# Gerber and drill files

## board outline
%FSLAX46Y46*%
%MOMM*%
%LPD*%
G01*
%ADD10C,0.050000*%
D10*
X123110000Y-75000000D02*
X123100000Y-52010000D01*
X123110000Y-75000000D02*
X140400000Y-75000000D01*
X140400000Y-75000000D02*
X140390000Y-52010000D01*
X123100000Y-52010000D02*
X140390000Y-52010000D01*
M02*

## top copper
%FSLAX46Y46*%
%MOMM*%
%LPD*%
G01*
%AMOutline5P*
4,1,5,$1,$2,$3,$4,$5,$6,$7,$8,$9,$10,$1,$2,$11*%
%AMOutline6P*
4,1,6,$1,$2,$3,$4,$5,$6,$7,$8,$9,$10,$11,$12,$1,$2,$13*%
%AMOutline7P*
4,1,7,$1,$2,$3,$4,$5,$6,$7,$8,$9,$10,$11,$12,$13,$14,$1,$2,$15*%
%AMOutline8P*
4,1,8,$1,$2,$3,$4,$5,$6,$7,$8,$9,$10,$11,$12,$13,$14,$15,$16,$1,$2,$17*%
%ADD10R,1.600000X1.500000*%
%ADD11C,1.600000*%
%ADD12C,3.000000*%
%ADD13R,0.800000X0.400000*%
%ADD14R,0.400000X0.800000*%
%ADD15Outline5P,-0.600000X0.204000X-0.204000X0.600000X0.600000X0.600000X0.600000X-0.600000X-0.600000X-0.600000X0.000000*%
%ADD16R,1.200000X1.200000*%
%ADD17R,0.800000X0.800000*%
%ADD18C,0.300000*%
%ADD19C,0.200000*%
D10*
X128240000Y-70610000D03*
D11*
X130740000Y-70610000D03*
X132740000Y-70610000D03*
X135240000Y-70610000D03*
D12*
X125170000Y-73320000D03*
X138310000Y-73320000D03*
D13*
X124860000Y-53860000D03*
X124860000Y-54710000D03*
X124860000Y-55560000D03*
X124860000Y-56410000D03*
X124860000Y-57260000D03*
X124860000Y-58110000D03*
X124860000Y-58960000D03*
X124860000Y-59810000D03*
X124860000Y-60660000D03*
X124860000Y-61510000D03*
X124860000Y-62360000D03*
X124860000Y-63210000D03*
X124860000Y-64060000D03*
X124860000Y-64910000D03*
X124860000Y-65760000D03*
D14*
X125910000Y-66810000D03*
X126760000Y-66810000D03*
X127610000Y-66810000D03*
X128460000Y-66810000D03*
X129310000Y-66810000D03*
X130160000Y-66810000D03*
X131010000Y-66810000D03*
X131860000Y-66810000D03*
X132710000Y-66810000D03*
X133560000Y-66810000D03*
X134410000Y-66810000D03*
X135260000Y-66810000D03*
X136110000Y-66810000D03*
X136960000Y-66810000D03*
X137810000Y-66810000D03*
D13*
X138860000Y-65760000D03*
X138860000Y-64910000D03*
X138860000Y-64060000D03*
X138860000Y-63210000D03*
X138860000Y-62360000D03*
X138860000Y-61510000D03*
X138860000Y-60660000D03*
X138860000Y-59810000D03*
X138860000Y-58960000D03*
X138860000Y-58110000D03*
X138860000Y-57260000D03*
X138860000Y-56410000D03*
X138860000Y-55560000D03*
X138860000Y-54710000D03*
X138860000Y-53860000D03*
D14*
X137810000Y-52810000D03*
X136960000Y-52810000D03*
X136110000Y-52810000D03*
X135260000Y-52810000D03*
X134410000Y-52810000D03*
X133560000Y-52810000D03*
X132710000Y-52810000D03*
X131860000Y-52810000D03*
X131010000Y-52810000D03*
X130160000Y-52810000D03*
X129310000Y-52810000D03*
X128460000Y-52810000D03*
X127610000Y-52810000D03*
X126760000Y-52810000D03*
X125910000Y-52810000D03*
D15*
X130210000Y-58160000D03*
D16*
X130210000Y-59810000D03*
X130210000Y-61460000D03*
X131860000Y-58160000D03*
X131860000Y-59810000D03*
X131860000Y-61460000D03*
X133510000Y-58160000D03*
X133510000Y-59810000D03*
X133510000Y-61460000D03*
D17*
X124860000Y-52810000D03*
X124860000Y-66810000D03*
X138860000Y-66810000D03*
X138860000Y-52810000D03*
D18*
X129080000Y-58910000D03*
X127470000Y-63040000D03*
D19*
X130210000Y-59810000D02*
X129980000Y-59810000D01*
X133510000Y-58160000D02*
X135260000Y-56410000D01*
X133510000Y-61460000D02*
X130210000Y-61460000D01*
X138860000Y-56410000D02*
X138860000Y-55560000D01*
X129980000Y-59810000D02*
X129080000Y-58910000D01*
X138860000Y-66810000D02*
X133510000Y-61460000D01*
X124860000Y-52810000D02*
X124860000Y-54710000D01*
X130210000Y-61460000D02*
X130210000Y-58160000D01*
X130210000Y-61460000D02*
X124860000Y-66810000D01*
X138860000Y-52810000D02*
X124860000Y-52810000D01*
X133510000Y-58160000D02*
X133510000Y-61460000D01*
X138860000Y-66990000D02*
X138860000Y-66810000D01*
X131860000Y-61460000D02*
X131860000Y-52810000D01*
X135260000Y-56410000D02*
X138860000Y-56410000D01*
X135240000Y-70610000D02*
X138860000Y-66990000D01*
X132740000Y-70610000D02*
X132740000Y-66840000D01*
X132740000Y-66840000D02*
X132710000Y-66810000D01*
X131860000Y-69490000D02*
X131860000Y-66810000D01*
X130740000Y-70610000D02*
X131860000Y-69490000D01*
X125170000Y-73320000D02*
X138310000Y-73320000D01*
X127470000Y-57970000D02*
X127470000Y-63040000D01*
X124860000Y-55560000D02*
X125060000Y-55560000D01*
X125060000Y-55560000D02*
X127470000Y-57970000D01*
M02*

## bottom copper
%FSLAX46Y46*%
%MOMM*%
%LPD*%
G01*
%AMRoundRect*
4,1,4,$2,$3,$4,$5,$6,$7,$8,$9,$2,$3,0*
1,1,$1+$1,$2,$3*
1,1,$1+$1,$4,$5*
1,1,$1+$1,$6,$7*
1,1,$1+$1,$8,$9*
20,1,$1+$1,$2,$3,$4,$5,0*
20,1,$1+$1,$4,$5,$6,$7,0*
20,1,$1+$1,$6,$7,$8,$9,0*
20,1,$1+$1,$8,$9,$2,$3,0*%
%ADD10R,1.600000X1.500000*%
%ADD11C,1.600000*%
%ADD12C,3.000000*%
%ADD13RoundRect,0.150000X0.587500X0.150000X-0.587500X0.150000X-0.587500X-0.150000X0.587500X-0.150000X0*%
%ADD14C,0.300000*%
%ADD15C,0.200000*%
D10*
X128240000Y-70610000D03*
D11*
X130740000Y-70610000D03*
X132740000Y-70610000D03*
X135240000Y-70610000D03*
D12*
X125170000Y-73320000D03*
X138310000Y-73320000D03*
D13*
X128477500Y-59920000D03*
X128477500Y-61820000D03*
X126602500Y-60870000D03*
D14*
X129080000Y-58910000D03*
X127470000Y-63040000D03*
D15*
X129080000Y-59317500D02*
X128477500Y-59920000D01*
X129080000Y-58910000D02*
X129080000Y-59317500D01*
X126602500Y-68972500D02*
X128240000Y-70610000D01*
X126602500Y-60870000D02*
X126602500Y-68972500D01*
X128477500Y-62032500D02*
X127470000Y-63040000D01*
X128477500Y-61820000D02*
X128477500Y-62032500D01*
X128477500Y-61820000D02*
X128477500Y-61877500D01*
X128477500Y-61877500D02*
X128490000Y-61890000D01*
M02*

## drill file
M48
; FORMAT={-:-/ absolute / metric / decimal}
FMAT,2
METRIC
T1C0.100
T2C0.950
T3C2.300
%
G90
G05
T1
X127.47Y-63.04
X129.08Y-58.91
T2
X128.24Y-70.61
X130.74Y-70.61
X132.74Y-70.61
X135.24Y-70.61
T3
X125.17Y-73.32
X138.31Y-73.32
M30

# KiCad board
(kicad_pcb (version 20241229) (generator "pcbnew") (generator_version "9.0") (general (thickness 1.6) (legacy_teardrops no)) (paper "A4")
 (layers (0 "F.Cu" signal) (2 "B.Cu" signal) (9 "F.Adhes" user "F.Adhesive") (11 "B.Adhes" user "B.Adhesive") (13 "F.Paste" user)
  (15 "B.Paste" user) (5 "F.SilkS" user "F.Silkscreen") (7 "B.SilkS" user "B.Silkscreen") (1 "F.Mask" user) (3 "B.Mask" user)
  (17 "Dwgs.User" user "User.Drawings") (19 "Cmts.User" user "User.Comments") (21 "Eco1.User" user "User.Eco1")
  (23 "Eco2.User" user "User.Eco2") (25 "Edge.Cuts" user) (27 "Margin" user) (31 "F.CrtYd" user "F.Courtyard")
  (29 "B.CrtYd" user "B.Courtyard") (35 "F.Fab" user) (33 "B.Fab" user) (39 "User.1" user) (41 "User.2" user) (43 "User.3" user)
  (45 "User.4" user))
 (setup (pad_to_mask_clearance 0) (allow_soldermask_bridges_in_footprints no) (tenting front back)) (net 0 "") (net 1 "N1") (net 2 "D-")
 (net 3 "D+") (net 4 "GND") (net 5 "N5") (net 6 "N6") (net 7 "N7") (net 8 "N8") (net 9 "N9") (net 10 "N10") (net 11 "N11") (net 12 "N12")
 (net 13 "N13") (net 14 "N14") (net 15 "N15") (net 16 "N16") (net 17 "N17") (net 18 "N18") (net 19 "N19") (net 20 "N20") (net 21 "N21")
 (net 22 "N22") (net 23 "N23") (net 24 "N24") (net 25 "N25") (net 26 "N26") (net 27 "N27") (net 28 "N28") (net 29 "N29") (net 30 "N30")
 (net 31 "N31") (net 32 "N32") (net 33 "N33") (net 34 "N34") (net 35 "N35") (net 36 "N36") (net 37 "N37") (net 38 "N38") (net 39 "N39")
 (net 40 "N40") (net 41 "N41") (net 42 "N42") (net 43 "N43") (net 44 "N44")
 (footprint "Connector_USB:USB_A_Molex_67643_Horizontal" (layer "F.Cu") (at 128.24 70.61)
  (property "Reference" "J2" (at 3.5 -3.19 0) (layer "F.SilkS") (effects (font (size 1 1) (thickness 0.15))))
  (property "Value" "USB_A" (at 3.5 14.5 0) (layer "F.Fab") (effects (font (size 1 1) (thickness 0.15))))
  (pad "1" thru_hole rect (at 0 0) (size 1.6 1.5) (drill 0.95) (layers "*.Cu" "*.Mask") (remove_unused_layers no) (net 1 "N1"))
  (pad "2" thru_hole circle (at 2.5 0) (size 1.6 1.6) (drill 0.95) (layers "*.Cu" "*.Mask") (remove_unused_layers no) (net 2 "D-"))
  (pad "3" thru_hole circle (at 4.5 0) (size 1.6 1.6) (drill 0.95) (layers "*.Cu" "*.Mask") (remove_unused_layers no) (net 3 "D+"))
  (pad "4" thru_hole circle (at 7 0) (size 1.6 1.6) (drill 0.95) (layers "*.Cu" "*.Mask") (remove_unused_layers no) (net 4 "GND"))
  (pad "5" thru_hole circle (at -3.07 2.71) (size 3 3) (drill 2.3) (layers "*.Cu" "*.Mask") (remove_unused_layers no) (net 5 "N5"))
  (pad "5" thru_hole circle (at 10.07 2.71) (size 3 3) (drill 2.3) (layers "*.Cu" "*.Mask") (remove_unused_layers no) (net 5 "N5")))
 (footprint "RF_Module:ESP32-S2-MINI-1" (layer "F.Cu") (at 131.86 57.26)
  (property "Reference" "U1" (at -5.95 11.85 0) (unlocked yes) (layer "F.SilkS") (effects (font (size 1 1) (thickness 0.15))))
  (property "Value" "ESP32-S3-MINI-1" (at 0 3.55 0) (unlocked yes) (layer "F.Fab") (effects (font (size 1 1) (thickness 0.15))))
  (pad "1" smd rect (at -7 -3.4) (size 0.8 0.4) (layers "F.Cu" "F.Mask" "F.Paste") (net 4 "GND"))
  (pad "2" smd rect (at -7 -2.55) (size 0.8 0.4) (layers "F.Cu" "F.Mask" "F.Paste") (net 4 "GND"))
  (pad "3" smd rect (at -7 -1.7) (size 0.8 0.4) (layers "F.Cu" "F.Mask" "F.Paste") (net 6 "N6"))
  (pad "4" smd rect (at -7 -0.85) (size 0.8 0.4) (layers "F.Cu" "F.Mask" "F.Paste") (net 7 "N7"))
  (pad "5" smd rect (at -7 0) (size 0.8 0.4) (layers "F.Cu" "F.Mask" "F.Paste") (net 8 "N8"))
  (pad "6" smd rect (at -7 0.85) (size 0.8 0.4) (layers "F.Cu" "F.Mask" "F.Paste") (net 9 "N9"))
  (pad "7" smd rect (at -7 1.7) (size 0.8 0.4) (layers "F.Cu" "F.Mask" "F.Paste") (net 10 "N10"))
  (pad "8" smd rect (at -7 2.55) (size 0.8 0.4) (layers "F.Cu" "F.Mask" "F.Paste") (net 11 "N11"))
  (pad "9" smd rect (at -7 3.4) (size 0.8 0.4) (layers "F.Cu" "F.Mask" "F.Paste") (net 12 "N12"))
  (pad "10" smd rect (at -7 4.25) (size 0.8 0.4) (layers "F.Cu" "F.Mask" "F.Paste") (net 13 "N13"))
  (pad "11" smd rect (at -7 5.1) (size 0.8 0.4) (layers "F.Cu" "F.Mask" "F.Paste") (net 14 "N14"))
  (pad "12" smd rect (at -7 5.95) (size 0.8 0.4) (layers "F.Cu" "F.Mask" "F.Paste") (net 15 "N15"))
  (pad "13" smd rect (at -7 6.8) (size 0.8 0.4) (layers "F.Cu" "F.Mask" "F.Paste") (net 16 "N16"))
  (pad "14" smd rect (at -7 7.65) (size 0.8 0.4) (layers "F.Cu" "F.Mask" "F.Paste") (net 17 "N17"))
  (pad "15" smd rect (at -7 8.5) (size 0.8 0.4) (layers "F.Cu" "F.Mask" "F.Paste") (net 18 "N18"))
  (pad "16" smd rect (at -5.95 9.55 90) (size 0.8 0.4) (layers "F.Cu" "F.Mask" "F.Paste") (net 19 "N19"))
  (pad "17" smd rect (at -5.1 9.55 90) (size 0.8 0.4) (layers "F.Cu" "F.Mask" "F.Paste") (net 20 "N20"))
  (pad "18" smd rect (at -4.25 9.55 90) (size 0.8 0.4) (layers "F.Cu" "F.Mask" "F.Paste") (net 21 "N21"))
  (pad "19" smd rect (at -3.4 9.55 90) (size 0.8 0.4) (layers "F.Cu" "F.Mask" "F.Paste") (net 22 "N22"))
  (pad "20" smd rect (at -2.55 9.55 90) (size 0.8 0.4) (layers "F.Cu" "F.Mask" "F.Paste") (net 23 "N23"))
  (pad "21" smd rect (at -1.7 9.55 90) (size 0.8 0.4) (layers "F.Cu" "F.Mask" "F.Paste") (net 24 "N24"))
  (pad "22" smd rect (at -0.85 9.55 90) (size 0.8 0.4) (layers "F.Cu" "F.Mask" "F.Paste") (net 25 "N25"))
  (pad "23" smd rect (at 0 9.55 90) (size 0.8 0.4) (layers "F.Cu" "F.Mask" "F.Paste") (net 2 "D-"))
  (pad "24" smd rect (at 0.85 9.55 90) (size 0.8 0.4) (layers "F.Cu" "F.Mask" "F.Paste") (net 3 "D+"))
  (pad "25" smd rect (at 1.7 9.55 90) (size 0.8 0.4) (layers "F.Cu" "F.Mask" "F.Paste") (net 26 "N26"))
  (pad "26" smd rect (at 2.55 9.55 90) (size 0.8 0.4) (layers "F.Cu" "F.Mask" "F.Paste") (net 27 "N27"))
  (pad "27" smd rect (at 3.4 9.55 90) (size 0.8 0.4) (layers "F.Cu" "F.Mask" "F.Paste") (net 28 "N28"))
  (pad "28" smd rect (at 4.25 9.55 90) (size 0.8 0.4) (layers "F.Cu" "F.Mask" "F.Paste") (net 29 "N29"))
  (pad "29" smd rect (at 5.1 9.55 90) (size 0.8 0.4) (layers "F.Cu" "F.Mask" "F.Paste") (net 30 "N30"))
  (pad "30" smd rect (at 5.95 9.55 90) (size 0.8 0.4) (layers "F.Cu" "F.Mask" "F.Paste") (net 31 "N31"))
  (pad "31" smd rect (at 7 8.5) (size 0.8 0.4) (layers "F.Cu" "F.Mask" "F.Paste") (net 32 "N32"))
  (pad "32" smd rect (at 7 7.65) (size 0.8 0.4) (layers "F.Cu" "F.Mask" "F.Paste") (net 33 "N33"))
  (pad "33" smd rect (at 7 6.8) (size 0.8 0.4) (layers "F.Cu" "F.Mask" "F.Paste") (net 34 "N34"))
  (pad "34" smd rect (at 7 5.95) (size 0.8 0.4) (layers "F.Cu" "F.Mask" "F.Paste") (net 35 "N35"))
  (pad "35" smd rect (at 7 5.1) (size 0.8 0.4) (layers "F.Cu" "F.Mask" "F.Paste") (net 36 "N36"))
  (pad "36" smd rect (at 7 4.25) (size 0.8 0.4) (layers "F.Cu" "F.Mask" "F.Paste") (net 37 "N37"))
  (pad "37" smd rect (at 7 3.4) (size 0.8 0.4) (layers "F.Cu" "F.Mask" "F.Paste") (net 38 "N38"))
  (pad "38" smd rect (at 7 2.55) (size 0.8 0.4) (layers "F.Cu" "F.Mask" "F.Paste") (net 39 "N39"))
  (pad "39" smd rect (at 7 1.7) (size 0.8 0.4) (layers "F.Cu" "F.Mask" "F.Paste") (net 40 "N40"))
  (pad "40" smd rect (at 7 0.85) (size 0.8 0.4) (layers "F.Cu" "F.Mask" "F.Paste") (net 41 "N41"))
  (pad "41" smd rect (at 7 0) (size 0.8 0.4) (layers "F.Cu" "F.Mask" "F.Paste") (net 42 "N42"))
  (pad "42" smd rect (at 7 -0.85) (size 0.8 0.4) (layers "F.Cu" "F.Mask" "F.Paste") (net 4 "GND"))
  (pad "43" smd rect (at 7 -1.7) (size 0.8 0.4) (layers "F.Cu" "F.Mask" "F.Paste") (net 4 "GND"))
  (pad "44" smd rect (at 7 -2.55) (size 0.8 0.4) (layers "F.Cu" "F.Mask" "F.Paste") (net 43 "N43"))
  (pad "45" smd rect (at 7 -3.4) (size 0.8 0.4) (layers "F.Cu" "F.Mask" "F.Paste") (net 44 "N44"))
  (pad "46" smd rect (at 5.95 -4.45 90) (size 0.8 0.4) (layers "F.Cu" "F.Mask" "F.Paste") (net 4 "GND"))
  (pad "47" smd rect (at 5.1 -4.45 90) (size 0.8 0.4) (layers "F.Cu" "F.Mask" "F.Paste") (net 4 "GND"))
  (pad "48" smd rect (at 4.25 -4.45 90) (size 0.8 0.4) (layers "F.Cu" "F.Mask" "F.Paste") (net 4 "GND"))
  (pad "49" smd rect (at 3.4 -4.45 90) (size 0.8 0.4) (layers "F.Cu" "F.Mask" "F.Paste") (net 4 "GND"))
  (pad "50" smd rect (at 2.55 -4.45 90) (size 0.8 0.4) (layers "F.Cu" "F.Mask" "F.Paste") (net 4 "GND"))
  (pad "51" smd rect (at 1.7 -4.45 90) (size 0.8 0.4) (layers "F.Cu" "F.Mask" "F.Paste") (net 4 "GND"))
  (pad "52" smd rect (at 0.85 -4.45 90) (size 0.8 0.4) (layers "F.Cu" "F.Mask" "F.Paste") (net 4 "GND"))
  (pad "53" smd rect (at 0 -4.45 90) (size 0.8 0.4) (layers "F.Cu" "F.Mask" "F.Paste") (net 4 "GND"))
  (pad "54" smd rect (at -0.85 -4.45 90) (size 0.8 0.4) (layers "F.Cu" "F.Mask" "F.Paste") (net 4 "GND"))
  (pad "55" smd rect (at -1.7 -4.45 90) (size 0.8 0.4) (layers "F.Cu" "F.Mask" "F.Paste") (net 4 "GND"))
  (pad "56" smd rect (at -2.55 -4.45 90) (size 0.8 0.4) (layers "F.Cu" "F.Mask" "F.Paste") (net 4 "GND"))
  (pad "57" smd rect (at -3.4 -4.45 90) (size 0.8 0.4) (layers "F.Cu" "F.Mask" "F.Paste") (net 4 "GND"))
  (pad "58" smd rect (at -4.25 -4.45 90) (size 0.8 0.4) (layers "F.Cu" "F.Mask" "F.Paste") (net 4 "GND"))
  (pad "59" smd rect (at -5.1 -4.45 90) (size 0.8 0.4) (layers "F.Cu" "F.Mask" "F.Paste") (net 4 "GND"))
  (pad "60" smd rect (at -5.95 -4.45 90) (size 0.8 0.4) (layers "F.Cu" "F.Mask" "F.Paste") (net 4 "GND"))
  (pad "61" smd roundrect (at -1.65 0.9) (size 1.2 1.2) (layers "F.Cu" "F.Mask" "F.Paste") (roundrect_rratio 0) (chamfer_ratio 0.33)
   (chamfer top_left) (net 4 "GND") (zone_connect 2))
  (pad "61" smd rect (at -1.65 2.55) (size 1.2 1.2) (layers "F.Cu" "F.Mask" "F.Paste") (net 4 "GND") (zone_connect 2))
  (pad "61" smd rect (at -1.65 4.2) (size 1.2 1.2) (layers "F.Cu" "F.Mask" "F.Paste") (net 4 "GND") (zone_connect 2))
  (pad "61" smd rect (at 0 0.9) (size 1.2 1.2) (layers "F.Cu" "F.Mask" "F.Paste") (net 4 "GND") (zone_connect 2))
  (pad "61" smd rect (at 0 2.55) (size 1.2 1.2) (layers "F.Cu" "F.Mask" "F.Paste") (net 4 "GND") (zone_connect 2))
  (pad "61" smd rect (at 0 4.2) (size 1.2 1.2) (layers "F.Cu" "F.Mask" "F.Paste") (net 4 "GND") (zone_connect 2))
  (pad "61" smd rect (at 1.65 0.9) (size 1.2 1.2) (layers "F.Cu" "F.Mask" "F.Paste") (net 4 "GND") (zone_connect 2))
  (pad "61" smd rect (at 1.65 2.55) (size 1.2 1.2) (layers "F.Cu" "F.Mask" "F.Paste") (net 4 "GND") (zone_connect 2))
  (pad "61" smd rect (at 1.65 4.2) (size 1.2 1.2) (layers "F.Cu" "F.Mask" "F.Paste") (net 4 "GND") (zone_connect 2))
  (pad "62" smd rect (at -7 -4.45) (size 0.8 0.8) (layers "F.Cu" "F.Mask" "F.Paste") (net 4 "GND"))
  (pad "63" smd rect (at -7 9.55) (size 0.8 0.8) (layers "F.Cu" "F.Mask" "F.Paste") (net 4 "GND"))
  (pad "64" smd rect (at 7 9.55) (size 0.8 0.8) (layers "F.Cu" "F.Mask" "F.Paste") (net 4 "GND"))
  (pad "65" smd rect (at 7 -4.45) (size 0.8 0.8) (layers "F.Cu" "F.Mask" "F.Paste") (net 4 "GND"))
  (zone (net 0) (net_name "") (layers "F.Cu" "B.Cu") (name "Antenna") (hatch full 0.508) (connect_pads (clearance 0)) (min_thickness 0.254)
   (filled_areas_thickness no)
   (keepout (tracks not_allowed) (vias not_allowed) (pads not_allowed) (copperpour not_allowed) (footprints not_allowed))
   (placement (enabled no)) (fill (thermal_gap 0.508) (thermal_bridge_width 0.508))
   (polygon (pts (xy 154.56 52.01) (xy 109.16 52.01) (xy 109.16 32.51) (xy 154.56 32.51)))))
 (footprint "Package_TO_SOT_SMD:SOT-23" (layer "B.Cu") (at 127.54 60.87 180)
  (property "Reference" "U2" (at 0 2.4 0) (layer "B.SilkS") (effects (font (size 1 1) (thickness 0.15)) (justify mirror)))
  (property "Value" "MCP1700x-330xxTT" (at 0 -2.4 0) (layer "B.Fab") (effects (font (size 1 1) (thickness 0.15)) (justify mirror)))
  (pad "1" smd roundrect (at -0.9375 0.95 180) (size 1.475 0.6) (layers "B.Cu" "B.Mask" "B.Paste") (roundrect_rratio 0.25) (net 4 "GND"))
  (pad "2" smd roundrect (at -0.9375 -0.95 180) (size 1.475 0.6) (layers "B.Cu" "B.Mask" "B.Paste") (roundrect_rratio 0.25) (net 6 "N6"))
  (pad "3" smd roundrect (at 0.9375 0 180) (size 1.475 0.6) (layers "B.Cu" "B.Mask" "B.Paste") (roundrect_rratio 0.25) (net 1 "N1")))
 (gr_line (start 123.11 75) (end 123.1 52.01) (stroke (width 0.05) (type default)) (layer "Edge.Cuts"))
 (gr_line (start 123.11 75) (end 140.4 75) (stroke (width 0.05) (type default)) (layer "Edge.Cuts"))
 (gr_line (start 140.4 75) (end 140.39 52.01) (stroke (width 0.05) (type default)) (layer "Edge.Cuts"))
 (gr_line (start 123.1 52.01) (end 140.39 52.01) (stroke (width 0.05) (type default)) (layer "Edge.Cuts"))
 (segment (start 130.21 59.81) (end 129.98 59.81) (width 0.2) (layer "F.Cu") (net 4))
 (segment (start 133.51 58.16) (end 135.26 56.41) (width 0.2) (layer "F.Cu") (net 4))
 (segment (start 133.51 61.46) (end 130.21 61.46) (width 0.2) (layer "F.Cu") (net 4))
 (segment (start 138.86 56.41) (end 138.86 55.56) (width 0.2) (layer "F.Cu") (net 4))
 (segment (start 129.98 59.81) (end 129.08 58.91) (width 0.2) (layer "F.Cu") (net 4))
 (segment (start 138.86 66.81) (end 133.51 61.46) (width 0.2) (layer "F.Cu") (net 4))
 (segment (start 124.86 52.81) (end 124.86 54.71) (width 0.2) (layer "F.Cu") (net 4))
 (segment (start 130.21 61.46) (end 130.21 58.16) (width 0.2) (layer "F.Cu") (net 4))
 (segment (start 130.21 61.46) (end 124.86 66.81) (width 0.2) (layer "F.Cu") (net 4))
 (segment (start 138.86 52.81) (end 124.86 52.81) (width 0.2) (layer "F.Cu") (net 4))
 (segment (start 133.51 58.16) (end 133.51 61.46) (width 0.2) (layer "F.Cu") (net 4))
 (segment (start 138.86 66.99) (end 138.86 66.81) (width 0.2) (layer "F.Cu") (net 4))
 (segment (start 131.86 61.46) (end 131.86 52.81) (width 0.2) (layer "F.Cu") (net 4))
 (segment (start 135.26 56.41) (end 138.86 56.41) (width 0.2) (layer "F.Cu") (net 4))
 (segment (start 135.24 70.61) (end 138.86 66.99) (width 0.2) (layer "F.Cu") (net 4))
 (via micro (at 129.08 58.91) (size 0.3) (drill 0.1) (layers "F.Cu" "B.Cu") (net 4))
 (segment (start 129.08 59.3175) (end 128.4775 59.92) (width 0.2) (layer "B.Cu") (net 4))
 (segment (start 129.08 58.91) (end 129.08 59.3175) (width 0.2) (layer "B.Cu") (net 4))
 (segment (start 126.6025 68.9725) (end 128.24 70.61) (width 0.2) (layer "B.Cu") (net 1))
 (segment (start 126.6025 60.87) (end 126.6025 68.9725) (width 0.2) (layer "B.Cu") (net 1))
 (segment (start 132.74 70.61) (end 132.74 66.84) (width 0.2) (layer "F.Cu") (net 3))
 (segment (start 132.74 66.84) (end 132.71 66.81) (width 0.2) (layer "F.Cu") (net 3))
 (segment (start 131.86 69.49) (end 131.86 66.81) (width 0.2) (layer "F.Cu") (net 2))
 (segment (start 130.74 70.61) (end 131.86 69.49) (width 0.2) (layer "F.Cu") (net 2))
 (segment (start 125.17 73.32) (end 138.31 73.32) (width 0.2) (layer "F.Cu") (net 5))
 (segment (start 127.47 57.97) (end 127.47 63.04) (width 0.2) (layer "F.Cu") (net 6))
 (segment (start 124.86 55.56) (end 125.06 55.56) (width 0.2) (layer "F.Cu") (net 6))
 (segment (start 125.06 55.56) (end 127.47 57.97) (width 0.2) (layer "F.Cu") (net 6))
 (via micro (at 127.47 63.04) (size 0.3) (drill 0.1) (layers "F.Cu" "B.Cu") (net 6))
 (segment (start 128.4775 62.0325) (end 127.47 63.04) (width 0.2) (layer "B.Cu") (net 6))
 (segment (start 128.4775 61.82) (end 128.4775 62.0325) (width 0.2) (layer "B.Cu") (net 6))
 (segment (start 128.4775 61.82) (end 128.4775 61.8775) (width 0.2) (layer "B.Cu") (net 6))
 (segment (start 128.4775 61.8775) (end 128.49 61.89) (width 0.2) (layer "B.Cu") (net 6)))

